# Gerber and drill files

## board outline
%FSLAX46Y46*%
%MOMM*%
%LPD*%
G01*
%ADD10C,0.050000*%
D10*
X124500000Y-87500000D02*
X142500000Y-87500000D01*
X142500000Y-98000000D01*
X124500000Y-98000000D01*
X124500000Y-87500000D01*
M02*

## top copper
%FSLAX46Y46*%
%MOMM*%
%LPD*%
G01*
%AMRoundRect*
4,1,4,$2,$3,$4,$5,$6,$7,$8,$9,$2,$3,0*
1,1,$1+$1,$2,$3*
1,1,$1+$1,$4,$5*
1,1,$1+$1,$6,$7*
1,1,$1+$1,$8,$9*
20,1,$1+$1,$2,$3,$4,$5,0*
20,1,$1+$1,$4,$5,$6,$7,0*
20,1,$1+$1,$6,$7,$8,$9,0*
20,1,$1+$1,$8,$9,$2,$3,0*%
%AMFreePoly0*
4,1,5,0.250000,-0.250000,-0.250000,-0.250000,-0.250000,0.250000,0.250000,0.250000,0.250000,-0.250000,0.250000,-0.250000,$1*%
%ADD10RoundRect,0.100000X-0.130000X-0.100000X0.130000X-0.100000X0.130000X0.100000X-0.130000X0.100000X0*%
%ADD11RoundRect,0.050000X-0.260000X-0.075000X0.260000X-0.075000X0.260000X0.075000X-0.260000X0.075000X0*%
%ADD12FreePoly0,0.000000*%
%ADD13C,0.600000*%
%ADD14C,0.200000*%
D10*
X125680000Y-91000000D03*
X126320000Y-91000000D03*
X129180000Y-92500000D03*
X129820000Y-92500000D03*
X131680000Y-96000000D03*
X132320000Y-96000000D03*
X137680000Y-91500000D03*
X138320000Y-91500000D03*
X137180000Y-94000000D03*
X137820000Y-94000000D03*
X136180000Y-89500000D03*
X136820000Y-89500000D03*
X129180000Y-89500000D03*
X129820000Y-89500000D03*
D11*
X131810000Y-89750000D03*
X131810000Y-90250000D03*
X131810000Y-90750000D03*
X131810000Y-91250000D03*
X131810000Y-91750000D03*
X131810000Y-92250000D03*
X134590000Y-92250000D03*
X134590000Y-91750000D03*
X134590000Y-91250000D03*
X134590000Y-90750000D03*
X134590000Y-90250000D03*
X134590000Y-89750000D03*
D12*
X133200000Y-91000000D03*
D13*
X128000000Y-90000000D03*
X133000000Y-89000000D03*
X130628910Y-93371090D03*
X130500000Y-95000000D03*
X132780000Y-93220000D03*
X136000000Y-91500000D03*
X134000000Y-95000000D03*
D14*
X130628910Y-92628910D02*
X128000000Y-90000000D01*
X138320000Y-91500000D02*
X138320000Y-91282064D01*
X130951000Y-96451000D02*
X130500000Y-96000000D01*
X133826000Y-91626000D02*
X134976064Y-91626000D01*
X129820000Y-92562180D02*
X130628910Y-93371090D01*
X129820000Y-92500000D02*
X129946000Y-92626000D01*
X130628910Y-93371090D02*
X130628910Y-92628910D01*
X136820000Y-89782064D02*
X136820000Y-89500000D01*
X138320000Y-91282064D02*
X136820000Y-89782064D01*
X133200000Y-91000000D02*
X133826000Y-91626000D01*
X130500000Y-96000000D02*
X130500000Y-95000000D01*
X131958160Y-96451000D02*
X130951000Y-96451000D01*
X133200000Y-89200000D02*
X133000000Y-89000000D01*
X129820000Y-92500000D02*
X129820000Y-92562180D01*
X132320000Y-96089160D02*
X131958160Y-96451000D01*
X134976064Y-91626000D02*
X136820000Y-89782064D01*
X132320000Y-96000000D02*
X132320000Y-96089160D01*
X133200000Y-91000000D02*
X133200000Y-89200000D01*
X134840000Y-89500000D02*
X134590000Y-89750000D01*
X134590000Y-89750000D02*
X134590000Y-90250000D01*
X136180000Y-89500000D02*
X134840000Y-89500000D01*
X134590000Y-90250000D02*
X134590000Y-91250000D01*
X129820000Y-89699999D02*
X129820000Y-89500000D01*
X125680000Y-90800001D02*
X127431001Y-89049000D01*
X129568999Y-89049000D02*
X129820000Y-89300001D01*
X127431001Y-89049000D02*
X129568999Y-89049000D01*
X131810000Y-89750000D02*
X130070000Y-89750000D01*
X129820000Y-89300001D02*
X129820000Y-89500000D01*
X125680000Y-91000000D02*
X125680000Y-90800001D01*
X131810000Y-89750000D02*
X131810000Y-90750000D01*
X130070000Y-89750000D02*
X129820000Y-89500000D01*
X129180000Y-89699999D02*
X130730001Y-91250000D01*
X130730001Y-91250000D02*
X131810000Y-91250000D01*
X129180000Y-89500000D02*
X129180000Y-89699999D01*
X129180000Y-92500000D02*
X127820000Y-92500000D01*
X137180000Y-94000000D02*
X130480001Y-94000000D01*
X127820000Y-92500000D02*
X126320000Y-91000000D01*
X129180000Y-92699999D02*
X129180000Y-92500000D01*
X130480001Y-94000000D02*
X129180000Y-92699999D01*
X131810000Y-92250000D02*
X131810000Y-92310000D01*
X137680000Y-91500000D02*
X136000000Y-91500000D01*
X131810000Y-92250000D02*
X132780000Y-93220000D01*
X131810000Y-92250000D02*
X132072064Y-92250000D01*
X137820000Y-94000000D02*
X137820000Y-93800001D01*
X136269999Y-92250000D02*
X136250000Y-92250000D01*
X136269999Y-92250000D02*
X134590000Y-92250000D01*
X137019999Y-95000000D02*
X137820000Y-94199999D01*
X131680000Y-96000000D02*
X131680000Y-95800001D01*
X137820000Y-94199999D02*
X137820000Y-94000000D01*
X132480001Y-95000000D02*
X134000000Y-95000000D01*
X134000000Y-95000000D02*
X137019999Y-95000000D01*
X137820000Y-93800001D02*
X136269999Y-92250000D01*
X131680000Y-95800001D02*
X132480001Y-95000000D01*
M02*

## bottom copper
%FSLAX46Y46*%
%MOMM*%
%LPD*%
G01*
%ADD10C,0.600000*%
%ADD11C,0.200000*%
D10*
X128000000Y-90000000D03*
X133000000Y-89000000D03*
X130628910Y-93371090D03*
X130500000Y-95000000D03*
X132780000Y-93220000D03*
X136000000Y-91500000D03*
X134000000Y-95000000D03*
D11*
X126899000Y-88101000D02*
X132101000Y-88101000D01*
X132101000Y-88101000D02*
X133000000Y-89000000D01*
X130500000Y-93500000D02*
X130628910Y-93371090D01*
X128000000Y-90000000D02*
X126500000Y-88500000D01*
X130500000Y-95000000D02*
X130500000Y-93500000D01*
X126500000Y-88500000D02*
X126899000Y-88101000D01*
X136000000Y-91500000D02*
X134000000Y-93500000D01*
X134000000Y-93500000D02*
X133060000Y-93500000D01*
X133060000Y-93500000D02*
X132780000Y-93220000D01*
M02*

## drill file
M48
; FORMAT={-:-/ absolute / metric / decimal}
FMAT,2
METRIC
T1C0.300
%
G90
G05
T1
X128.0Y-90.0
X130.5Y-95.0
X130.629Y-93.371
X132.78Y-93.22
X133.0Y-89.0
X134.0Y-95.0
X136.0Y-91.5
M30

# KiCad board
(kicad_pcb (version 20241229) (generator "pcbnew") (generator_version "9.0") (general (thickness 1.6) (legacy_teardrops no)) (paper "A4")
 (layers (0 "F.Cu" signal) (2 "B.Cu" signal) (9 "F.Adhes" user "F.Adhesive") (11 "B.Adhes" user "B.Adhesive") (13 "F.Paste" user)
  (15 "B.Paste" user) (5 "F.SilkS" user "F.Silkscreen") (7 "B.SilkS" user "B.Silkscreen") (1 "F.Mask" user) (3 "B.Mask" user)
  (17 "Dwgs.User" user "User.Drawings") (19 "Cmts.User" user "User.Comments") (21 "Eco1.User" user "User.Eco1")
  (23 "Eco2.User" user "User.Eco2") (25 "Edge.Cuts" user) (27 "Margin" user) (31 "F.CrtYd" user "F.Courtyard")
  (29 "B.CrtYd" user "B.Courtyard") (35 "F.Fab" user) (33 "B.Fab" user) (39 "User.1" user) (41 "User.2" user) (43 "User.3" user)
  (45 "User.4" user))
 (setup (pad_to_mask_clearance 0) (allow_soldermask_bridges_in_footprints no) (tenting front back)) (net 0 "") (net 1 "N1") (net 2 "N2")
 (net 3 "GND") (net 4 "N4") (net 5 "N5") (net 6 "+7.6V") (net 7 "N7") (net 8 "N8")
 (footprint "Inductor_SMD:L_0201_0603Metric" (layer "F.Cu") (at 126 91)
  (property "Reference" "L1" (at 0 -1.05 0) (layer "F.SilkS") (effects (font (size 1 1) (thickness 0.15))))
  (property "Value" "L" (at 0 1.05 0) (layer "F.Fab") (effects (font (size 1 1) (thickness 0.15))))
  (pad "" smd roundrect (at -0.345 0) (size 0.318 0.36) (layers "F.Paste") (roundrect_rratio 0.25))
  (pad "" smd roundrect (at 0.345 0) (size 0.318 0.36) (layers "F.Paste") (roundrect_rratio 0.25))
  (pad "1" smd roundrect (at -0.32 0) (size 0.46 0.4) (layers "F.Cu" "F.Mask") (roundrect_rratio 0.25) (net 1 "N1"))
  (pad "2" smd roundrect (at 0.32 0) (size 0.46 0.4) (layers "F.Cu" "F.Mask") (roundrect_rratio 0.25) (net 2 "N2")))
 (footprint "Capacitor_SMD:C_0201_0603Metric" (layer "F.Cu") (at 129.5 92.5)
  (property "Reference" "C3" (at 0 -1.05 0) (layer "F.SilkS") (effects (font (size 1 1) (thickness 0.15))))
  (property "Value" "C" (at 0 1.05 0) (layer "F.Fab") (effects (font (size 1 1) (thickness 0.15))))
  (pad "" smd roundrect (at -0.345 0) (size 0.318 0.36) (layers "F.Paste") (roundrect_rratio 0.25))
  (pad "" smd roundrect (at 0.345 0) (size 0.318 0.36) (layers "F.Paste") (roundrect_rratio 0.25))
  (pad "1" smd roundrect (at -0.32 0) (size 0.46 0.4) (layers "F.Cu" "F.Mask") (roundrect_rratio 0.25) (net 2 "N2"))
  (pad "2" smd roundrect (at 0.32 0) (size 0.46 0.4) (layers "F.Cu" "F.Mask") (roundrect_rratio 0.25) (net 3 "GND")))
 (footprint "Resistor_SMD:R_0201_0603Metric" (layer "F.Cu") (at 132 96)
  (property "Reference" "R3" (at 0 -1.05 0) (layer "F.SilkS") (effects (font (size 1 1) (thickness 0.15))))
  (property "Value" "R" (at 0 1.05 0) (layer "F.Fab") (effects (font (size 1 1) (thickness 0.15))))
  (pad "" smd roundrect (at -0.345 0) (size 0.318 0.36) (layers "F.Paste") (roundrect_rratio 0.25))
  (pad "" smd roundrect (at 0.345 0) (size 0.318 0.36) (layers "F.Paste") (roundrect_rratio 0.25))
  (pad "1" smd roundrect (at -0.32 0) (size 0.46 0.4) (layers "F.Cu" "F.Mask") (roundrect_rratio 0.25) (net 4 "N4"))
  (pad "2" smd roundrect (at 0.32 0) (size 0.46 0.4) (layers "F.Cu" "F.Mask") (roundrect_rratio 0.25) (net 3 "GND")))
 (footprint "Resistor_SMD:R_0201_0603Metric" (layer "F.Cu") (at 138 91.5)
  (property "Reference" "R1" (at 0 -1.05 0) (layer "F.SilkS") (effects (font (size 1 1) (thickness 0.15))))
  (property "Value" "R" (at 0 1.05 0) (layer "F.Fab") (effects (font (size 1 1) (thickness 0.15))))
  (pad "" smd roundrect (at -0.345 0) (size 0.318 0.36) (layers "F.Paste") (roundrect_rratio 0.25))
  (pad "" smd roundrect (at 0.345 0) (size 0.318 0.36) (layers "F.Paste") (roundrect_rratio 0.25))
  (pad "1" smd roundrect (at -0.32 0) (size 0.46 0.4) (layers "F.Cu" "F.Mask") (roundrect_rratio 0.25) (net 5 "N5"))
  (pad "2" smd roundrect (at 0.32 0) (size 0.46 0.4) (layers "F.Cu" "F.Mask") (roundrect_rratio 0.25) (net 3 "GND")))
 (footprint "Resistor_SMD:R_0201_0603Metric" (layer "F.Cu") (at 137.5 94)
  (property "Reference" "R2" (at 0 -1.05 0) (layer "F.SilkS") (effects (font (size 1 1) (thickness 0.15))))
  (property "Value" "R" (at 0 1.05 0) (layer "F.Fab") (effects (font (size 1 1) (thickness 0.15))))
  (pad "" smd roundrect (at -0.345 0) (size 0.318 0.36) (layers "F.Paste") (roundrect_rratio 0.25))
  (pad "" smd roundrect (at 0.345 0) (size 0.318 0.36) (layers "F.Paste") (roundrect_rratio 0.25))
  (pad "1" smd roundrect (at -0.32 0) (size 0.46 0.4) (layers "F.Cu" "F.Mask") (roundrect_rratio 0.25) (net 2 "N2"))
  (pad "2" smd roundrect (at 0.32 0) (size 0.46 0.4) (layers "F.Cu" "F.Mask") (roundrect_rratio 0.25) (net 4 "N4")))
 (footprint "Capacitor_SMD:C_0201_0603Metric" (layer "F.Cu") (at 136.5 89.5)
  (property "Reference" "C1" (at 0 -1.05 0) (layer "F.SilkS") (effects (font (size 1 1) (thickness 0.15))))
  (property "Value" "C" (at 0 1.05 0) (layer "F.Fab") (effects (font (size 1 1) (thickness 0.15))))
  (pad "" smd roundrect (at -0.345 0) (size 0.318 0.36) (layers "F.Paste") (roundrect_rratio 0.25))
  (pad "" smd roundrect (at 0.345 0) (size 0.318 0.36) (layers "F.Paste") (roundrect_rratio 0.25))
  (pad "1" smd roundrect (at -0.32 0) (size 0.46 0.4) (layers "F.Cu" "F.Mask") (roundrect_rratio 0.25) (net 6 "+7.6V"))
  (pad "2" smd roundrect (at 0.32 0) (size 0.46 0.4) (layers "F.Cu" "F.Mask") (roundrect_rratio 0.25) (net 3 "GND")))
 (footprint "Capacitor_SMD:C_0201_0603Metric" (layer "F.Cu") (at 129.5 89.5)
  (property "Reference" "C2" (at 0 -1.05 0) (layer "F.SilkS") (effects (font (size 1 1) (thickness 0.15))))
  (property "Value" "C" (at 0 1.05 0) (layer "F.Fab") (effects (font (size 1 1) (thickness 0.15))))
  (pad "" smd roundrect (at -0.345 0) (size 0.318 0.36) (layers "F.Paste") (roundrect_rratio 0.25))
  (pad "" smd roundrect (at 0.345 0) (size 0.318 0.36) (layers "F.Paste") (roundrect_rratio 0.25))
  (pad "1" smd roundrect (at -0.32 0) (size 0.46 0.4) (layers "F.Cu" "F.Mask") (roundrect_rratio 0.25) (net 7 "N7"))
  (pad "2" smd roundrect (at 0.32 0) (size 0.46 0.4) (layers "F.Cu" "F.Mask") (roundrect_rratio 0.25) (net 1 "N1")))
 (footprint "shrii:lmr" (layer "F.Cu") (at 139.5 94)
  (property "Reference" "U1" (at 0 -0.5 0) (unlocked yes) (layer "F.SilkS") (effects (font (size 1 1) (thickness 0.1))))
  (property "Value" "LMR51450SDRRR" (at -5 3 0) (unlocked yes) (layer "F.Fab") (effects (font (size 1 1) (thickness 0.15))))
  (pad "1" smd roundrect (at -7.69 -4.25) (size 0.62 0.25) (layers "F.Cu" "F.Paste") (roundrect_rratio 0.2) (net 1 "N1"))
  (pad "2" smd roundrect (at -7.69 -3.75) (size 0.62 0.25) (layers "F.Cu" "F.Paste") (roundrect_rratio 0.2) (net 1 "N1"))
  (pad "3" smd roundrect (at -7.69 -3.25) (size 0.62 0.25) (layers "F.Cu" "F.Paste") (roundrect_rratio 0.2) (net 1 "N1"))
  (pad "4" smd roundrect (at -7.69 -2.75) (size 0.62 0.25) (layers "F.Cu" "F.Paste") (roundrect_rratio 0.2) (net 7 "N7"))
  (pad "5" smd roundrect (at -7.69 -2.25) (size 0.62 0.25) (layers "F.Cu" "F.Paste") (roundrect_rratio 0.2) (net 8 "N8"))
  (pad "6" smd roundrect (at -7.69 -1.75) (size 0.62 0.25) (layers "F.Cu" "F.Paste") (roundrect_rratio 0.2) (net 5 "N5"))
  (pad "7" smd roundrect (at -4.91 -1.75) (size 0.62 0.25) (layers "F.Cu" "F.Paste") (roundrect_rratio 0.2) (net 4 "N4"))
  (pad "8" smd roundrect (at -4.91 -2.25) (size 0.62 0.25) (layers "F.Cu" "F.Paste") (roundrect_rratio 0.2) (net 3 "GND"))
  (pad "9" smd roundrect (at -4.91 -2.75) (size 0.62 0.25) (layers "F.Cu" "F.Paste") (roundrect_rratio 0.2) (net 6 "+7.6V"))
  (pad "10" smd roundrect (at -4.91 -3.25) (size 0.62 0.25) (layers "F.Cu" "F.Paste") (roundrect_rratio 0.2) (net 6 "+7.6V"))
  (pad "11" smd roundrect (at -4.91 -3.75) (size 0.62 0.25) (layers "F.Cu" "F.Paste") (roundrect_rratio 0.2) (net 6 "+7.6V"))
  (pad "12" smd roundrect (at -4.91 -4.25) (size 0.62 0.25) (layers "F.Cu" "F.Paste") (roundrect_rratio 0.2) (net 6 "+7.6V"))
  (pad "13" smd custom (at -6.3 -3) (size 0.5 0.5) (layers "F.Cu") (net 3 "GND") (zone_connect 2)
   (options (clearance outline) (anchor rect)) (primitives)))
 (gr_rect (start 124.5 87.5) (end 142.5 98) (stroke (width 0.05) (type default)) (fill no) (layer "Edge.Cuts"))
 (segment (start 130.62891 92.62891) (end 128 90) (width 0.2) (layer "F.Cu") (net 3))
 (segment (start 138.32 91.5) (end 138.32 91.282064) (width 0.2) (layer "F.Cu") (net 3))
 (segment (start 130.951 96.451) (end 130.5 96) (width 0.2) (layer "F.Cu") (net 3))
 (segment (start 133.826 91.626) (end 134.976064 91.626) (width 0.2) (layer "F.Cu") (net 3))
 (segment (start 129.82 92.56218) (end 130.62891 93.37109) (width 0.2) (layer "F.Cu") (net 3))
 (segment (start 129.82 92.5) (end 129.946 92.626) (width 0.2) (layer "F.Cu") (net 3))
 (segment (start 130.62891 93.37109) (end 130.62891 92.62891) (width 0.2) (layer "F.Cu") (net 3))
 (segment (start 136.82 89.782064) (end 136.82 89.5) (width 0.2) (layer "F.Cu") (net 3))
 (segment (start 138.32 91.282064) (end 136.82 89.782064) (width 0.2) (layer "F.Cu") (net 3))
 (segment (start 133.2 91) (end 133.826 91.626) (width 0.2) (layer "F.Cu") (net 3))
 (segment (start 130.5 96) (end 130.5 95) (width 0.2) (layer "F.Cu") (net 3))
 (segment (start 131.95816 96.451) (end 130.951 96.451) (width 0.2) (layer "F.Cu") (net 3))
 (segment (start 133.2 89.2) (end 133 89) (width 0.2) (layer "F.Cu") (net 3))
 (segment (start 129.82 92.5) (end 129.82 92.56218) (width 0.2) (layer "F.Cu") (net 3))
 (segment (start 132.32 96.08916) (end 131.95816 96.451) (width 0.2) (layer "F.Cu") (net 3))
 (segment (start 134.976064 91.626) (end 136.82 89.782064) (width 0.2) (layer "F.Cu") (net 3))
 (segment (start 132.32 96) (end 132.32 96.08916) (width 0.2) (layer "F.Cu") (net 3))
 (segment (start 133.2 91) (end 133.2 89.2) (width 0.2) (layer "F.Cu") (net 3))
 (via (at 128 90) (size 0.6) (drill 0.3) (layers "F.Cu" "B.Cu") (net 3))
 (via (at 133 89) (size 0.6) (drill 0.3) (layers "F.Cu" "B.Cu") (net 3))
 (via (at 130.62891 93.37109) (size 0.6) (drill 0.3) (layers "F.Cu" "B.Cu") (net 3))
 (via (at 130.5 95) (size 0.6) (drill 0.3) (layers "F.Cu" "B.Cu") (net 3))
 (segment (start 126.899 88.101) (end 132.101 88.101) (width 0.2) (layer "B.Cu") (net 3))
 (segment (start 132.101 88.101) (end 133 89) (width 0.2) (layer "B.Cu") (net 3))
 (segment (start 130.5 93.5) (end 130.62891 93.37109) (width 0.2) (layer "B.Cu") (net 3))
 (segment (start 128 90) (end 126.5 88.5) (width 0.2) (layer "B.Cu") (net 3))
 (segment (start 130.5 95) (end 130.5 93.5) (width 0.2) (layer "B.Cu") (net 3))
 (segment (start 126.5 88.5) (end 126.899 88.101) (width 0.2) (layer "B.Cu") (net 3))
 (segment (start 134.84 89.5) (end 134.59 89.75) (width 0.2) (layer "F.Cu") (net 6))
 (segment (start 134.59 89.75) (end 134.59 90.25) (width 0.2) (layer "F.Cu") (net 6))
 (segment (start 136.18 89.5) (end 134.84 89.5) (width 0.2) (layer "F.Cu") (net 6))
 (segment (start 134.59 90.25) (end 134.59 91.25) (width 0.2) (layer "F.Cu") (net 6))
 (segment (start 129.82 89.699999) (end 129.82 89.5) (width 0.2) (layer "F.Cu") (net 1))
 (segment (start 125.68 90.800001) (end 127.431001 89.049) (width 0.2) (layer "F.Cu") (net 1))
 (segment (start 129.568999 89.049) (end 129.82 89.300001) (width 0.2) (layer "F.Cu") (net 1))
 (segment (start 127.431001 89.049) (end 129.568999 89.049) (width 0.2) (layer "F.Cu") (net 1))
 (segment (start 131.81 89.75) (end 130.07 89.75) (width 0.2) (layer "F.Cu") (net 1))
 (segment (start 129.82 89.300001) (end 129.82 89.5) (width 0.2) (layer "F.Cu") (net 1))
 (segment (start 125.68 91) (end 125.68 90.800001) (width 0.2) (layer "F.Cu") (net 1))
 (segment (start 131.81 89.75) (end 131.81 90.75) (width 0.2) (layer "F.Cu") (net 1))
 (segment (start 130.07 89.75) (end 129.82 89.5) (width 0.2) (layer "F.Cu") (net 1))
 (segment (start 129.18 89.699999) (end 130.730001 91.25) (width 0.2) (layer "F.Cu") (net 7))
 (segment (start 130.730001 91.25) (end 131.81 91.25) (width 0.2) (layer "F.Cu") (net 7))
 (segment (start 129.18 89.5) (end 129.18 89.699999) (width 0.2) (layer "F.Cu") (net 7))
 (segment (start 129.18 92.5) (end 127.82 92.5) (width 0.2) (layer "F.Cu") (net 2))
 (segment (start 137.18 94) (end 130.480001 94) (width 0.2) (layer "F.Cu") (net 2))
 (segment (start 127.82 92.5) (end 126.32 91) (width 0.2) (layer "F.Cu") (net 2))
 (segment (start 129.18 92.699999) (end 129.18 92.5) (width 0.2) (layer "F.Cu") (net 2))
 (segment (start 130.480001 94) (end 129.18 92.699999) (width 0.2) (layer "F.Cu") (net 2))
 (segment (start 131.81 92.25) (end 131.81 92.31) (width 0.2) (layer "F.Cu") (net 5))
 (segment (start 137.68 91.5) (end 136 91.5) (width 0.2) (layer "F.Cu") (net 5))
 (segment (start 131.81 92.25) (end 132.78 93.22) (width 0.2) (layer "F.Cu") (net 5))
 (segment (start 131.81 92.25) (end 132.072064 92.25) (width 0.2) (layer "F.Cu") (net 5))
 (via (at 132.78 93.22) (size 0.6) (drill 0.3) (layers "F.Cu" "B.Cu") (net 5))
 (via (at 136 91.5) (size 0.6) (drill 0.3) (layers "F.Cu" "B.Cu") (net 5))
 (segment (start 136 91.5) (end 134 93.5) (width 0.2) (layer "B.Cu") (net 5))
 (segment (start 134 93.5) (end 133.06 93.5) (width 0.2) (layer "B.Cu") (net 5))
 (segment (start 133.06 93.5) (end 132.78 93.22) (width 0.2) (layer "B.Cu") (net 5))
 (segment (start 137.82 94) (end 137.82 93.800001) (width 0.2) (layer "F.Cu") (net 4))
 (segment (start 136.269999 92.25) (end 136.25 92.25) (width 0.2) (layer "F.Cu") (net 4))
 (segment (start 136.269999 92.25) (end 134.59 92.25) (width 0.2) (layer "F.Cu") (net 4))
 (segment (start 137.019999 95) (end 137.82 94.199999) (width 0.2) (layer "F.Cu") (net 4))
 (segment (start 131.68 96) (end 131.68 95.800001) (width 0.2) (layer "F.Cu") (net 4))
 (segment (start 137.82 94.199999) (end 137.82 94) (width 0.2) (layer "F.Cu") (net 4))
 (segment (start 132.480001 95) (end 134 95) (width 0.2) (layer "F.Cu") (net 4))
 (segment (start 134 95) (end 137.019999 95) (width 0.2) (layer "F.Cu") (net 4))
 (segment (start 137.82 93.800001) (end 136.269999 92.25) (width 0.2) (layer "F.Cu") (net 4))
 (segment (start 131.68 95.800001) (end 132.480001 95) (width 0.2) (layer "F.Cu") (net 4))
 (via (at 134 95) (size 0.6) (drill 0.3) (layers "F.Cu" "B.Cu") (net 4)))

